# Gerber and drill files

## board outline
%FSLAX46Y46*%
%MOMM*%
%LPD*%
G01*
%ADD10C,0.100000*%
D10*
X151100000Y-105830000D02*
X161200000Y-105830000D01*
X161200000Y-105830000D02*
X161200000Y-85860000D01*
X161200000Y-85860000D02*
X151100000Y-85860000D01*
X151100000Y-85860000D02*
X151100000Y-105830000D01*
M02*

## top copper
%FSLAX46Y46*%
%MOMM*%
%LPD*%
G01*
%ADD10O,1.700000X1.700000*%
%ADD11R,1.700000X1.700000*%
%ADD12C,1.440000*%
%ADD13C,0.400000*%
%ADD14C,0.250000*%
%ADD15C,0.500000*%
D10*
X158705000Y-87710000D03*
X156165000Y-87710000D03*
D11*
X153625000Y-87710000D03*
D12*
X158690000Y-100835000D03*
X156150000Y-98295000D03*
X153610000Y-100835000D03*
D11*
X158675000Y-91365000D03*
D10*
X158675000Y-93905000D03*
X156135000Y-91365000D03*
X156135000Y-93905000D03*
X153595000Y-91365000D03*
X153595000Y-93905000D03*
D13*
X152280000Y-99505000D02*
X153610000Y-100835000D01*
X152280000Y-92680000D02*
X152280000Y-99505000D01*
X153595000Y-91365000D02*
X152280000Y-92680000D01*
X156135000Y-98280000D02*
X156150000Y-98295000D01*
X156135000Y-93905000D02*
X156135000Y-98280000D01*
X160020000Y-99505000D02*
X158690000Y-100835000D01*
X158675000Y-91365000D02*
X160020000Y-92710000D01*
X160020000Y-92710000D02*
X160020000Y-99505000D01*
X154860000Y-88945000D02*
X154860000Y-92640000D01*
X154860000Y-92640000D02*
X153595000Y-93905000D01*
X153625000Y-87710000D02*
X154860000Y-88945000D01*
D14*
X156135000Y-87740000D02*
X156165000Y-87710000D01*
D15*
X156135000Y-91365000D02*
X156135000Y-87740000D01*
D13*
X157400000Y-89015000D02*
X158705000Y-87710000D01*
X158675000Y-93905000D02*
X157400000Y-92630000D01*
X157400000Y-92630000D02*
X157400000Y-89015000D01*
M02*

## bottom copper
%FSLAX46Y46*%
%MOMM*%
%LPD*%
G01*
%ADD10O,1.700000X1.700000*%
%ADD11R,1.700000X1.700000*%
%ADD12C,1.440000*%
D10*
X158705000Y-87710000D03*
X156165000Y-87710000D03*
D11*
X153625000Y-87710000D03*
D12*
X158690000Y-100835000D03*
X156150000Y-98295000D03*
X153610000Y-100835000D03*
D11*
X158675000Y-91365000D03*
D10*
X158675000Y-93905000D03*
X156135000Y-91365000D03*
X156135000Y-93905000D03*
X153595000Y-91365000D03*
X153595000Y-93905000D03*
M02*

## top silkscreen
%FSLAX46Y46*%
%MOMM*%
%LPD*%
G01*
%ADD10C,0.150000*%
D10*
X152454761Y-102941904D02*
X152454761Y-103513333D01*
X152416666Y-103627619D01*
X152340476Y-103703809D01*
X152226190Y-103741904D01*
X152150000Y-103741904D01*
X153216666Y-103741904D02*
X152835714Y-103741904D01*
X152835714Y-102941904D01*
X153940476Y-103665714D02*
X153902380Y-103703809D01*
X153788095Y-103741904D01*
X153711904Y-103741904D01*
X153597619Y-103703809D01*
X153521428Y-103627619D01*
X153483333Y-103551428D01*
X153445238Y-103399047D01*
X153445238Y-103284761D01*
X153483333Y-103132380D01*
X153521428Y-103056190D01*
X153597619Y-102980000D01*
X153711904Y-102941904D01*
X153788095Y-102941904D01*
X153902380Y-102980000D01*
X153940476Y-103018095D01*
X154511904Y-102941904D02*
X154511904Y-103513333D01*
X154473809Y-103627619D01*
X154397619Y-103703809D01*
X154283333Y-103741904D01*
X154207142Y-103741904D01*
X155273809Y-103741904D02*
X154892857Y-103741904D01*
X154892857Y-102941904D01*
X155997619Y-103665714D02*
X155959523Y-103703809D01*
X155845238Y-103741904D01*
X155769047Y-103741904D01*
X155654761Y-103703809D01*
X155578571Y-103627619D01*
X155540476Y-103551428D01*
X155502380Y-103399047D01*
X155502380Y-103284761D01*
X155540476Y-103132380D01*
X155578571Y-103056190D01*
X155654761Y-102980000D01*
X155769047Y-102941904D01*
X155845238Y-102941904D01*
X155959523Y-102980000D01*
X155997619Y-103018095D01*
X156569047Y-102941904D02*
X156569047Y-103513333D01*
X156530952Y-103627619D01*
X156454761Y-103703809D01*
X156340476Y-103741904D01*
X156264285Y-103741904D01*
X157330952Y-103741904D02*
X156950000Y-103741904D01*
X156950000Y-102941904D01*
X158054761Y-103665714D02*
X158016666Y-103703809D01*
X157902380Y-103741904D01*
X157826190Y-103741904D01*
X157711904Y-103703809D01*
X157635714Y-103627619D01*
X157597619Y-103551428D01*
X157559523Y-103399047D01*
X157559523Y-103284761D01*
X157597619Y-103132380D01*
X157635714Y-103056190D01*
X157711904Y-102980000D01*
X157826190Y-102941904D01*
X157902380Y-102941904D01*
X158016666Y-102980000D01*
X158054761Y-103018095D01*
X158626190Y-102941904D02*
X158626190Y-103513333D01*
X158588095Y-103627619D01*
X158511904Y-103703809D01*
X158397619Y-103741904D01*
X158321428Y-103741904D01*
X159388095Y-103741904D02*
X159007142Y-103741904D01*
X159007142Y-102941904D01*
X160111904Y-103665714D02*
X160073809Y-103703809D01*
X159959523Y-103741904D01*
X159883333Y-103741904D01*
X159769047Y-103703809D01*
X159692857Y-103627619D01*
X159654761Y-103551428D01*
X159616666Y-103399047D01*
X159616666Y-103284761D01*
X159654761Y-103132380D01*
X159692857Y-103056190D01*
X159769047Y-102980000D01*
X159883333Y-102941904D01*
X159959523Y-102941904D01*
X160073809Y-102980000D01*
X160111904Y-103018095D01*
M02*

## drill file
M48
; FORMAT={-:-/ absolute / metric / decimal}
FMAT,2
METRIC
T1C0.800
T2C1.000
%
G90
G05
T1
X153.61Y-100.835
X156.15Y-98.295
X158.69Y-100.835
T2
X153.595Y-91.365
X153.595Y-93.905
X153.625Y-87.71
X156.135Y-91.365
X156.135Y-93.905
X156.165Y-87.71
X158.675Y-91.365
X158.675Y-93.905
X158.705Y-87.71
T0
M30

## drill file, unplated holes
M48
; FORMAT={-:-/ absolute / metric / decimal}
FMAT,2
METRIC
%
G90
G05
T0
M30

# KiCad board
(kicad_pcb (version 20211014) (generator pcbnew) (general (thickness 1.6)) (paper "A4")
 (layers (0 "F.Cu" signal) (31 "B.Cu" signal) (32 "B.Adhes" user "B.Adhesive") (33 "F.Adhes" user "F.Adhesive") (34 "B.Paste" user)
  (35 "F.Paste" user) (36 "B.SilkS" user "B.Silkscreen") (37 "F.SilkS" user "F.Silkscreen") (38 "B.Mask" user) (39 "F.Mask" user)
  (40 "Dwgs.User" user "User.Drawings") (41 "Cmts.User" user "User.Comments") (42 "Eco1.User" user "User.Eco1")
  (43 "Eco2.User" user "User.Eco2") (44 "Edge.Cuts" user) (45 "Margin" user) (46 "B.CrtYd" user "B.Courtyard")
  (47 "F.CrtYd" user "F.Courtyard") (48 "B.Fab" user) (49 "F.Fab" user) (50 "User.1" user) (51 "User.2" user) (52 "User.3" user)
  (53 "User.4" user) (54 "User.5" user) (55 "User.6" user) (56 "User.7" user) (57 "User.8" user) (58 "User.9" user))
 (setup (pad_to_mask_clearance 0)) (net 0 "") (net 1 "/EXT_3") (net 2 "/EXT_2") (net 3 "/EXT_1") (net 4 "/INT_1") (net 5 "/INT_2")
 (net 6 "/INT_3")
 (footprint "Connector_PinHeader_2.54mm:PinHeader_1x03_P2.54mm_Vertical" (layer "F.Cu") (at 153.625 87.71 90)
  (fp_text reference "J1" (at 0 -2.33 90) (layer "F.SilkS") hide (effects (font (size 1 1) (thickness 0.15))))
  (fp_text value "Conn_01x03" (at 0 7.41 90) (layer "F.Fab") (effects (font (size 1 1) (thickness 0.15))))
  (pad "1" thru_hole oval (at 0 5.08 90) (size 1.7 1.7) (drill 1) (layers *.Cu *.Mask) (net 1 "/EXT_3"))
  (pad "2" thru_hole oval (at 0 2.54 90) (size 1.7 1.7) (drill 1) (layers *.Cu *.Mask) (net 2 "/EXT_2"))
  (pad "3" thru_hole rect (at 0 0 90) (size 1.7 1.7) (drill 1) (layers *.Cu *.Mask) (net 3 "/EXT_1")))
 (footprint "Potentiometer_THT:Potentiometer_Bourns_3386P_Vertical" (layer "F.Cu") (at 158.69 100.835 90)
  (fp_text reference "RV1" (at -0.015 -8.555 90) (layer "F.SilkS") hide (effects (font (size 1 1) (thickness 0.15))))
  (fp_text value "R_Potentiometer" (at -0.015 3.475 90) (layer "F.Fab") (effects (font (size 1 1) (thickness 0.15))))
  (pad "1" thru_hole circle (at 0 0 90) (size 1.44 1.44) (drill 0.8) (layers *.Cu *.Mask) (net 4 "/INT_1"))
  (pad "2" thru_hole circle (at 2.54 -2.54 90) (size 1.44 1.44) (drill 0.8) (layers *.Cu *.Mask) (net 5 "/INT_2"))
  (pad "3" thru_hole circle (at 0 -5.08 90) (size 1.44 1.44) (drill 0.8) (layers *.Cu *.Mask) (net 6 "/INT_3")))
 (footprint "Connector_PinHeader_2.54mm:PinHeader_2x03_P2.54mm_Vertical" (layer "F.Cu") (at 158.675 91.365 -90)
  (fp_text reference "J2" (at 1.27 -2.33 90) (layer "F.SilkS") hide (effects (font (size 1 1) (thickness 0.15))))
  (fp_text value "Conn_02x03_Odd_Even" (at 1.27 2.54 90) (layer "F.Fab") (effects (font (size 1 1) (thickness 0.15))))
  (pad "1" thru_hole rect (at 0 0 270) (size 1.7 1.7) (drill 1) (layers *.Cu *.Mask) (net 4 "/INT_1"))
  (pad "2" thru_hole oval (at 2.54 0 270) (size 1.7 1.7) (drill 1) (layers *.Cu *.Mask) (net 1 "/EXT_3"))
  (pad "3" thru_hole oval (at 0 2.54 270) (size 1.7 1.7) (drill 1) (layers *.Cu *.Mask) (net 2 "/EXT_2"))
  (pad "4" thru_hole oval (at 2.54 2.54 270) (size 1.7 1.7) (drill 1) (layers *.Cu *.Mask) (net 5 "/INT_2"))
  (pad "5" thru_hole oval (at 0 5.08 270) (size 1.7 1.7) (drill 1) (layers *.Cu *.Mask) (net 6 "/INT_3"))
  (pad "6" thru_hole oval (at 2.54 5.08 270) (size 1.7 1.7) (drill 1) (layers *.Cu *.Mask) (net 3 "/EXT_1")))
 (gr_rect (start 151.1 105.83) (end 161.2 85.86) (layer "Edge.Cuts") (width 0.1) (fill none))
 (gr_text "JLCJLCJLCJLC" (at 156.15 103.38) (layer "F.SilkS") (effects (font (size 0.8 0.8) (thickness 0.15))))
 (segment (start 152.28 99.505) (end 153.61 100.835) (width 0.4) (layer "F.Cu") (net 6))
 (segment (start 152.28 92.68) (end 152.28 99.505) (width 0.4) (layer "F.Cu") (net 6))
 (segment (start 153.595 91.365) (end 152.28 92.68) (width 0.4) (layer "F.Cu") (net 6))
 (segment (start 156.135 98.28) (end 156.15 98.295) (width 0.4) (layer "F.Cu") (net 5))
 (segment (start 156.135 93.905) (end 156.135 98.28) (width 0.4) (layer "F.Cu") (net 5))
 (segment (start 160.02 99.505) (end 158.69 100.835) (width 0.4) (layer "F.Cu") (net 4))
 (segment (start 158.675 91.365) (end 160.02 92.71) (width 0.4) (layer "F.Cu") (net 4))
 (segment (start 160.02 92.71) (end 160.02 99.505) (width 0.4) (layer "F.Cu") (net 4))
 (segment (start 154.86 88.945) (end 154.86 92.64) (width 0.4) (layer "F.Cu") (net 3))
 (segment (start 154.86 92.64) (end 153.595 93.905) (width 0.4) (layer "F.Cu") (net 3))
 (segment (start 153.625 87.71) (end 154.86 88.945) (width 0.4) (layer "F.Cu") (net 3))
 (segment (start 156.135 87.74) (end 156.165 87.71) (width 0.25) (layer "F.Cu") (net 2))
 (segment (start 156.135 91.365) (end 156.135 87.74) (width 0.5) (layer "F.Cu") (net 2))
 (segment (start 157.4 89.015) (end 158.705 87.71) (width 0.4) (layer "F.Cu") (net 1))
 (segment (start 158.675 93.905) (end 157.4 92.63) (width 0.4) (layer "F.Cu") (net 1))
 (segment (start 157.4 92.63) (end 157.4 89.015) (width 0.4) (layer "F.Cu") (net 1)))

